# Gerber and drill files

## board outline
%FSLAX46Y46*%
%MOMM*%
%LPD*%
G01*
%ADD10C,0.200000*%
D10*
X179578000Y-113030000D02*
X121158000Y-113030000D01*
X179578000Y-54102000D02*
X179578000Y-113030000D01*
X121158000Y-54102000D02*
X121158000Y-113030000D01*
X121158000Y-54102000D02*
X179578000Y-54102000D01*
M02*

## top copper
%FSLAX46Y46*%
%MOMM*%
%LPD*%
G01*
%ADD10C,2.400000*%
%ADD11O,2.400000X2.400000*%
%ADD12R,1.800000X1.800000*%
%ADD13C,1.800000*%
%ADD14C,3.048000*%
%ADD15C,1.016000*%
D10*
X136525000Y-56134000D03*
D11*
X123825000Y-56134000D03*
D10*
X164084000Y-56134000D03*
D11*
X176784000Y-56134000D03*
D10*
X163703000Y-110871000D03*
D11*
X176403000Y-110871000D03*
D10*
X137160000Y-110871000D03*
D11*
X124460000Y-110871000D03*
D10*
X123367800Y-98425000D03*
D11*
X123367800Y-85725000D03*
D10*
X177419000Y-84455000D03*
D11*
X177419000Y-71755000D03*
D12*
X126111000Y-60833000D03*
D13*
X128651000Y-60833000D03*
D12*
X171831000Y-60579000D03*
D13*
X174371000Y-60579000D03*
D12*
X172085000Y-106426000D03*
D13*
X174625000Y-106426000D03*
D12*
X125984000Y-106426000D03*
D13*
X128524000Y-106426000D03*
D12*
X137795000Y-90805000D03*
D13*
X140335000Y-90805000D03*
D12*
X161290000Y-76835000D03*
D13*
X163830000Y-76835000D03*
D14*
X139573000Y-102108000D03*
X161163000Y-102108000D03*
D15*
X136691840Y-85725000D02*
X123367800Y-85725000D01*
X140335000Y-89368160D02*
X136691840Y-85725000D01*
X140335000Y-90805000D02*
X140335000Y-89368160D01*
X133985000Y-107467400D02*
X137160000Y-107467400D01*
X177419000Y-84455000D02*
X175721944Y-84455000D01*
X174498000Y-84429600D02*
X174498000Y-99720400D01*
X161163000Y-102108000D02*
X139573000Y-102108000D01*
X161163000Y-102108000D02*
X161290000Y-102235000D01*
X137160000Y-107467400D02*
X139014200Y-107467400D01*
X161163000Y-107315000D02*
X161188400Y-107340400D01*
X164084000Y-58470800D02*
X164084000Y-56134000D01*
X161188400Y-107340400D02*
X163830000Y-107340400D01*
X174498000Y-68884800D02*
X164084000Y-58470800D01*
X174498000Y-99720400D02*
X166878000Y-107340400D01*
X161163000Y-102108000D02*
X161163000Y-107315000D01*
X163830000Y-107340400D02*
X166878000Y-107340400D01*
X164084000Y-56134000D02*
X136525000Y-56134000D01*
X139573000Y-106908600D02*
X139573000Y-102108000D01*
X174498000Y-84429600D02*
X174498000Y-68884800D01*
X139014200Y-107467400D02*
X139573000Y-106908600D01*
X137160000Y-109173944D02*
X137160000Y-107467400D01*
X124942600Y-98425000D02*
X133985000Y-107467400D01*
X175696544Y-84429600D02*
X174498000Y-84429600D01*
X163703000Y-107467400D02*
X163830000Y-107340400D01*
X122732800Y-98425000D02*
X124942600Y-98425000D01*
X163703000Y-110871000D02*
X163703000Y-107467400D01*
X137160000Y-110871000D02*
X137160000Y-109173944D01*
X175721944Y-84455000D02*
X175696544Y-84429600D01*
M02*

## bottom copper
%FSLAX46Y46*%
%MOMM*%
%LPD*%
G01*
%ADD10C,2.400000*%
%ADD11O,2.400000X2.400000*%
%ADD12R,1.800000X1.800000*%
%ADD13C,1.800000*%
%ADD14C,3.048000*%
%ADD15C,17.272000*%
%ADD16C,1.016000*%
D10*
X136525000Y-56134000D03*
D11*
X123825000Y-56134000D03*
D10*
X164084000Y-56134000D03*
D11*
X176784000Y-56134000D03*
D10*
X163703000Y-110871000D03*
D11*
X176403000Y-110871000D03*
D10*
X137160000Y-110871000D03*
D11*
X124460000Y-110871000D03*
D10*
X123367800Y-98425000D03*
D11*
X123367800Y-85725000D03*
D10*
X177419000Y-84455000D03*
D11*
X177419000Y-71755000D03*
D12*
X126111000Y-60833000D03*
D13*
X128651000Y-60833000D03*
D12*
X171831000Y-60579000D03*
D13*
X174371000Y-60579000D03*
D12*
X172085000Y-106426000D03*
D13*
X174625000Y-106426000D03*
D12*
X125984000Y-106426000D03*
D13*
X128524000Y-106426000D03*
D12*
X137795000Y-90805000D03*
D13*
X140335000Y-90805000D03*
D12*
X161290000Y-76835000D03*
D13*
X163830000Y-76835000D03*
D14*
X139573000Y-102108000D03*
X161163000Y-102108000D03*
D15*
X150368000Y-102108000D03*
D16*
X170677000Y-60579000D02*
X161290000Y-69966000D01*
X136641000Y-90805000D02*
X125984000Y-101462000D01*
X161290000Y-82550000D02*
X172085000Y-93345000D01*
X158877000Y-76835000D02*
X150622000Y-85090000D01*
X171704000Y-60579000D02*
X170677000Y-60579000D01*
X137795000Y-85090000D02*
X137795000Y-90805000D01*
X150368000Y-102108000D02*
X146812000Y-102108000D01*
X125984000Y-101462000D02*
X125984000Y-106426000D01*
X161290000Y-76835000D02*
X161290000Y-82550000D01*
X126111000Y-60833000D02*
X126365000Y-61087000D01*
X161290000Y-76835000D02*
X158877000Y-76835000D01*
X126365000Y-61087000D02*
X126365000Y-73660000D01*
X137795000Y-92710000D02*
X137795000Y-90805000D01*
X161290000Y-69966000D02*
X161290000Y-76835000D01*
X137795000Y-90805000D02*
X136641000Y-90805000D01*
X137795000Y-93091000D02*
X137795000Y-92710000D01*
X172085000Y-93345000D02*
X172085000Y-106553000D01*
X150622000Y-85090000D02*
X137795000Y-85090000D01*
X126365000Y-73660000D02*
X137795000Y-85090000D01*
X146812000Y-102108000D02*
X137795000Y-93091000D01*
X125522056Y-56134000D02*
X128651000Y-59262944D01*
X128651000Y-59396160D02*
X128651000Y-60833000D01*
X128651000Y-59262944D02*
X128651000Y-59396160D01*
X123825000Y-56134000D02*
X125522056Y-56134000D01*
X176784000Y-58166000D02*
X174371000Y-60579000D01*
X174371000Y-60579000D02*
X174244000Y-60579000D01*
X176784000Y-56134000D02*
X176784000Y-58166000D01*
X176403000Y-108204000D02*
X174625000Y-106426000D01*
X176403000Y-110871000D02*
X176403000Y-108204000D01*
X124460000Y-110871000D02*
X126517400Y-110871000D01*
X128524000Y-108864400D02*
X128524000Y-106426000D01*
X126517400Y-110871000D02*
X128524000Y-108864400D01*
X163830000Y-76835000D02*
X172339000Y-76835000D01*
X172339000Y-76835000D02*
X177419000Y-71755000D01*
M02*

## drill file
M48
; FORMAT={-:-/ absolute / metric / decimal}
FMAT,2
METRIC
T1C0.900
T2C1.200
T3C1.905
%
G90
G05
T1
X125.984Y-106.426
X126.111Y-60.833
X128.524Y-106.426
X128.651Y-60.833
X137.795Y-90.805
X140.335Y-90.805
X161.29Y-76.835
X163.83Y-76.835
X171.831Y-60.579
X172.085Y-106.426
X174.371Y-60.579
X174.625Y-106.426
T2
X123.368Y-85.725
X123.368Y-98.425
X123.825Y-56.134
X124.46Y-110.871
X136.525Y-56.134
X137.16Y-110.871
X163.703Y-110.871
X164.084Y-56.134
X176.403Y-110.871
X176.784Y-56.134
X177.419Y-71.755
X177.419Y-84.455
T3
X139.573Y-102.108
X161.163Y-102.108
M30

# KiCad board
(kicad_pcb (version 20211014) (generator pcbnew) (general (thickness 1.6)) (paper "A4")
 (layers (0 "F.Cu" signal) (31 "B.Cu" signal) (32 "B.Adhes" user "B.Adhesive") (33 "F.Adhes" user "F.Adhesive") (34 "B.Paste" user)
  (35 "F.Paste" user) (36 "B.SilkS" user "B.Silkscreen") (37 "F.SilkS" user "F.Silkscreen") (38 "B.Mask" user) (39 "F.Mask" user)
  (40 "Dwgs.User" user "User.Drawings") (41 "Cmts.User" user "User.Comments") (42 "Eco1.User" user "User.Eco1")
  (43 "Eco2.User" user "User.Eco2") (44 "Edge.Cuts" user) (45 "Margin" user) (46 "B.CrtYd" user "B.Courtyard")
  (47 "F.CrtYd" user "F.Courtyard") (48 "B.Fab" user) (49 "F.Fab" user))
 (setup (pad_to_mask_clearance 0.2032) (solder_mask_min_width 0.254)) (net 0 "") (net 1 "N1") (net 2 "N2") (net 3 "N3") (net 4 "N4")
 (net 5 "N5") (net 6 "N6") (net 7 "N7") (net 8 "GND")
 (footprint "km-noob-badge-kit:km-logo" (layer "F.Cu") (at 150.368 83.566)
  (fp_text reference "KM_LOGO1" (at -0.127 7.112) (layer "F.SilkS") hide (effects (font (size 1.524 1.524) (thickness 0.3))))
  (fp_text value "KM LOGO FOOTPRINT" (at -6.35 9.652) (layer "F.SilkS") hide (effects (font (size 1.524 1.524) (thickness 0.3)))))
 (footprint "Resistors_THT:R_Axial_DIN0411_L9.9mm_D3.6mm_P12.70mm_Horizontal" (layer "F.Cu") (at 136.525 56.134 180)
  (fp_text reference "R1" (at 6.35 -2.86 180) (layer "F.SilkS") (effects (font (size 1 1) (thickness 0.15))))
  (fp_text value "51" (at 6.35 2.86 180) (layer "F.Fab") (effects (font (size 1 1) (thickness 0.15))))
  (pad "1" thru_hole circle locked (at 0 0 180) (size 2.4 2.4) (drill 1.2) (layers *.Cu *.Mask) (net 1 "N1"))
  (pad "2" thru_hole oval locked (at 12.7 0 180) (size 2.4 2.4) (drill 1.2) (layers *.Cu *.Mask) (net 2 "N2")))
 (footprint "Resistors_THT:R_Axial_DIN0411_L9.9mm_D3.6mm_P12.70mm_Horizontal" (layer "F.Cu") (at 164.084 56.134)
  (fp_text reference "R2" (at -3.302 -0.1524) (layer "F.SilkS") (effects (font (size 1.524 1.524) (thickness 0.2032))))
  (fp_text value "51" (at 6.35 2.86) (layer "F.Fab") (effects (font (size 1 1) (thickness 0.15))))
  (pad "1" thru_hole circle locked (at 0 0) (size 2.4 2.4) (drill 1.2) (layers *.Cu *.Mask) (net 1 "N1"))
  (pad "2" thru_hole oval locked (at 12.7 0) (size 2.4 2.4) (drill 1.2) (layers *.Cu *.Mask) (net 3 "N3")))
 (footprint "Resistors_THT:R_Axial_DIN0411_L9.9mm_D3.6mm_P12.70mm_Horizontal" (layer "F.Cu") (at 163.703 110.871)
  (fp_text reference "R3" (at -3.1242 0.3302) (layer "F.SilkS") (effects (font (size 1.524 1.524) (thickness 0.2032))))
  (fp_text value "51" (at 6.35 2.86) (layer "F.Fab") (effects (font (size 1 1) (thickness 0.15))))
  (pad "1" thru_hole circle locked (at 0 0) (size 2.4 2.4) (drill 1.2) (layers *.Cu *.Mask) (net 1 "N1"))
  (pad "2" thru_hole oval locked (at 12.7 0) (size 2.4 2.4) (drill 1.2) (layers *.Cu *.Mask) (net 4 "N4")))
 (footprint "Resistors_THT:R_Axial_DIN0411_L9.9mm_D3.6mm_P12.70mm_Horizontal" (layer "F.Cu") (at 137.16 110.871 180)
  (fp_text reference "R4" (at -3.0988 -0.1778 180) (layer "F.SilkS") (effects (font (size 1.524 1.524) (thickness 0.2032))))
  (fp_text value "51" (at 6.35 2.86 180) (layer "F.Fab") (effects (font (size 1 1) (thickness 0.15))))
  (pad "1" thru_hole circle locked (at 0 0 180) (size 2.4 2.4) (drill 1.2) (layers *.Cu *.Mask) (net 1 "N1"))
  (pad "2" thru_hole oval locked (at 12.7 0 180) (size 2.4 2.4) (drill 1.2) (layers *.Cu *.Mask) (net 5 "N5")))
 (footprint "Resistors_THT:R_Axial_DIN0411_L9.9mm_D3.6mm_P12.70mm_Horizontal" (layer "F.Cu") (at 123.3678 98.425 90)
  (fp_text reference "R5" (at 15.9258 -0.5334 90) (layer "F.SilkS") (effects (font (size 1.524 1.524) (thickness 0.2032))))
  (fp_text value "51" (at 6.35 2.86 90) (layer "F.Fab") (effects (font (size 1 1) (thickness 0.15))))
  (pad "1" thru_hole circle locked (at 0 0 90) (size 2.4 2.4) (drill 1.2) (layers *.Cu *.Mask) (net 1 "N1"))
  (pad "2" thru_hole oval locked (at 12.7 0 90) (size 2.4 2.4) (drill 1.2) (layers *.Cu *.Mask) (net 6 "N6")))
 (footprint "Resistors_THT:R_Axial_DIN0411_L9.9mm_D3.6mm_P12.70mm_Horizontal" (layer "F.Cu") (at 177.419 84.455 90)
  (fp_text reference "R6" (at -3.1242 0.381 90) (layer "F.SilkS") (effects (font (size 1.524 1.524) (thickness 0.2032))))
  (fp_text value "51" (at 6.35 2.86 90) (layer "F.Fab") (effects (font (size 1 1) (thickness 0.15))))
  (pad "1" thru_hole circle locked (at 0 0 90) (size 2.4 2.4) (drill 1.2) (layers *.Cu *.Mask) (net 1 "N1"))
  (pad "2" thru_hole oval locked (at 12.7 0 90) (size 2.4 2.4) (drill 1.2) (layers *.Cu *.Mask) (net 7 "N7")))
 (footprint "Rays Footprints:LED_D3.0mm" (layer "F.Cu") (at 126.111 60.833)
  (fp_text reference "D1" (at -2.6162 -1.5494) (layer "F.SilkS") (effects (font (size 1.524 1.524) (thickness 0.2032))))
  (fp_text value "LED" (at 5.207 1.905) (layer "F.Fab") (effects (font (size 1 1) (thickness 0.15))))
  (pad "1" thru_hole rect locked (at 0 0) (size 1.8 1.8) (drill 0.9) (layers *.Cu *.Mask) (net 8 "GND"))
  (pad "2" thru_hole circle locked (at 2.54 0) (size 1.8 1.8) (drill 0.9) (layers *.Cu *.Mask) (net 2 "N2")))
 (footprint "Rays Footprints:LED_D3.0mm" (layer "F.Cu") (at 171.831 60.579)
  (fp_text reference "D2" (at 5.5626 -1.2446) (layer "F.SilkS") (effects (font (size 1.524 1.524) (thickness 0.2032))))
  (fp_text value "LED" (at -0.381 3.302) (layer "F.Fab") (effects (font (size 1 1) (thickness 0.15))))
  (pad "1" thru_hole rect locked (at 0 0) (size 1.8 1.8) (drill 0.9) (layers *.Cu *.Mask) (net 8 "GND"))
  (pad "2" thru_hole circle locked (at 2.54 0) (size 1.8 1.8) (drill 0.9) (layers *.Cu *.Mask) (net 3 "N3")))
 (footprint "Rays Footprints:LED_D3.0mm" (layer "F.Cu") (at 172.085 106.426)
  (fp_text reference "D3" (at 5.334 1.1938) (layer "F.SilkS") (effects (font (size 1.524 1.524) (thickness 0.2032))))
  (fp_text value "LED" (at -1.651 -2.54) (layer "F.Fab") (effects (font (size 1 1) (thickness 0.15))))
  (pad "1" thru_hole rect locked (at 0 0) (size 1.8 1.8) (drill 0.9) (layers *.Cu *.Mask) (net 8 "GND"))
  (pad "2" thru_hole circle locked (at 2.54 0) (size 1.8 1.8) (drill 0.9) (layers *.Cu *.Mask) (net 4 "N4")))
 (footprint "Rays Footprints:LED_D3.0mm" (layer "F.Cu") (at 125.984 106.426)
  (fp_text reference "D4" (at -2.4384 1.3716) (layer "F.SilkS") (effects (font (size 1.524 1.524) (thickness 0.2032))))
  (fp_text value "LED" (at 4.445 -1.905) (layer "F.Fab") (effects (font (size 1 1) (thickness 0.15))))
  (pad "1" thru_hole rect locked (at 0 0) (size 1.8 1.8) (drill 0.9) (layers *.Cu *.Mask) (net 8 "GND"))
  (pad "2" thru_hole circle locked (at 2.54 0) (size 1.8 1.8) (drill 0.9) (layers *.Cu *.Mask) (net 5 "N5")))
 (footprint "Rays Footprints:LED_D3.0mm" (layer "F.Cu") (at 137.795 90.805)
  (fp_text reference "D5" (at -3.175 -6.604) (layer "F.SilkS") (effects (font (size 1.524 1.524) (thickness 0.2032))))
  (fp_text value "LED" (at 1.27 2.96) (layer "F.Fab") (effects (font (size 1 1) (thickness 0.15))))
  (pad "1" thru_hole rect locked (at 0 0) (size 1.8 1.8) (drill 0.9) (layers *.Cu *.Mask) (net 8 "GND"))
  (pad "2" thru_hole circle locked (at 2.54 0) (size 1.8 1.8) (drill 0.9) (layers *.Cu *.Mask) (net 6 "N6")))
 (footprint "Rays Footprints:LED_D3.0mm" (layer "F.Cu") (at 161.29 76.835)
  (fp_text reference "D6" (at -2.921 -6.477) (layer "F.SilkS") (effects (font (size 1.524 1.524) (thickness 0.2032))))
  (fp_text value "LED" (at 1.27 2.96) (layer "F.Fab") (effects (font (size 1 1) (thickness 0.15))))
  (pad "1" thru_hole rect locked (at 0 0) (size 1.8 1.8) (drill 0.9) (layers *.Cu *.Mask) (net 8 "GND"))
  (pad "2" thru_hole circle locked (at 2.54 0) (size 1.8 1.8) (drill 0.9) (layers *.Cu *.Mask) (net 7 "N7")))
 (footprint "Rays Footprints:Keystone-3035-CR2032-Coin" (layer "B.Cu") (at 150.368 102.108 180)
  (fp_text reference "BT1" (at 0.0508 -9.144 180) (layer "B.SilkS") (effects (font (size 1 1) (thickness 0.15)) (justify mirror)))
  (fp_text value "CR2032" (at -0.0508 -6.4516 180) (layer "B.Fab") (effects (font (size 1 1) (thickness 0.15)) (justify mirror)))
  (pad "1" thru_hole circle locked (at 10.795 0 180) (size 3.048 3.048) (drill 1.905) (layers *.Cu *.Mask) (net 1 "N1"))
  (pad "1" thru_hole circle locked (at -10.795 0 90) (size 3.048 3.048) (drill 1.905) (layers *.Cu *.Mask) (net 1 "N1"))
  (pad "2" smd circle locked (at 0 0 180) (size 17.272 17.272) (layers "B.Cu" "B.Paste" "B.Mask") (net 8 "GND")))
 (gr_line (start 179.578 113.03) (end 121.158 113.03) (layer "Edge.Cuts") (width 0.2))
 (gr_line (start 179.578 54.102) (end 179.578 113.03) (layer "Edge.Cuts") (width 0.2))
 (gr_line (start 121.158 54.102) (end 121.158 113.03) (layer "Edge.Cuts") (width 0.2))
 (gr_line (start 121.158 54.102) (end 179.578 54.102) (layer "Edge.Cuts") (width 0.2))
 (segment (start 170.677 60.579) (end 161.29 69.966) (width 1.016) (layer "B.Cu") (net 8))
 (segment (start 136.641 90.805) (end 125.984 101.462) (width 1.016) (layer "B.Cu") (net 8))
 (segment (start 161.29 82.55) (end 172.085 93.345) (width 1.016) (layer "B.Cu") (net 8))
 (segment (start 158.877 76.835) (end 150.622 85.09) (width 1.016) (layer "B.Cu") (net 8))
 (segment (start 171.704 60.579) (end 170.677 60.579) (width 1.016) (layer "B.Cu") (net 8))
 (segment (start 137.795 85.09) (end 137.795 90.805) (width 1.016) (layer "B.Cu") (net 8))
 (segment (start 150.368 102.108) (end 146.812 102.108) (width 1.016) (layer "B.Cu") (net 8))
 (segment (start 125.984 101.462) (end 125.984 106.426) (width 1.016) (layer "B.Cu") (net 8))
 (segment (start 161.29 76.835) (end 161.29 82.55) (width 1.016) (layer "B.Cu") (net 8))
 (segment (start 126.111 60.833) (end 126.365 61.087) (width 1.016) (layer "B.Cu") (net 8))
 (segment (start 161.29 76.835) (end 158.877 76.835) (width 1.016) (layer "B.Cu") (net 8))
 (segment (start 126.365 61.087) (end 126.365 73.66) (width 1.016) (layer "B.Cu") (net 8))
 (segment (start 137.795 92.71) (end 137.795 90.805) (width 1.016) (layer "B.Cu") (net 8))
 (segment (start 161.29 69.966) (end 161.29 76.835) (width 1.016) (layer "B.Cu") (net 8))
 (segment (start 137.795 90.805) (end 136.641 90.805) (width 1.016) (layer "B.Cu") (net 8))
 (segment (start 137.795 93.091) (end 137.795 92.71) (width 1.016) (layer "B.Cu") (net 8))
 (segment (start 172.085 93.345) (end 172.085 106.553) (width 1.016) (layer "B.Cu") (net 8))
 (segment (start 150.622 85.09) (end 137.795 85.09) (width 1.016) (layer "B.Cu") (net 8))
 (segment (start 126.365 73.66) (end 137.795 85.09) (width 1.016) (layer "B.Cu") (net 8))
 (segment (start 146.812 102.108) (end 137.795 93.091) (width 1.016) (layer "B.Cu") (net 8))
 (segment (start 125.522056 56.134) (end 128.651 59.262944) (width 1.016) (layer "B.Cu") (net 2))
 (segment (start 128.651 59.39616) (end 128.651 60.833) (width 1.016) (layer "B.Cu") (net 2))
 (segment (start 128.651 59.262944) (end 128.651 59.39616) (width 1.016) (layer "B.Cu") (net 2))
 (segment (start 123.825 56.134) (end 125.522056 56.134) (width 1.016) (layer "B.Cu") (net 2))
 (segment (start 176.784 58.166) (end 174.371 60.579) (width 1.016) (layer "B.Cu") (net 3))
 (segment (start 174.371 60.579) (end 174.244 60.579) (width 1.016) (layer "B.Cu") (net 3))
 (segment (start 176.784 56.134) (end 176.784 58.166) (width 1.016) (layer "B.Cu") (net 3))
 (segment (start 176.403 108.204) (end 174.625 106.426) (width 1.016) (layer "B.Cu") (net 4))
 (segment (start 176.403 110.871) (end 176.403 108.204) (width 1.016) (layer "B.Cu") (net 4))
 (segment (start 124.46 110.871) (end 126.5174 110.871) (width 1.016) (layer "B.Cu") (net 5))
 (segment (start 128.524 108.8644) (end 128.524 106.426) (width 1.016) (layer "B.Cu") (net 5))
 (segment (start 126.5174 110.871) (end 128.524 108.8644) (width 1.016) (layer "B.Cu") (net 5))
 (segment (start 136.69184 85.725) (end 123.3678 85.725) (width 1.016) (layer "F.Cu") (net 6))
 (segment (start 140.335 89.36816) (end 136.69184 85.725) (width 1.016) (layer "F.Cu") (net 6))
 (segment (start 140.335 90.805) (end 140.335 89.36816) (width 1.016) (layer "F.Cu") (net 6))
 (segment (start 163.83 76.835) (end 172.339 76.835) (width 1.016) (layer "B.Cu") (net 7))
 (segment (start 172.339 76.835) (end 177.419 71.755) (width 1.016) (layer "B.Cu") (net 7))
 (segment (start 133.985 107.4674) (end 137.16 107.4674) (width 1.016) (layer "F.Cu") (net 1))
 (segment (start 177.419 84.455) (end 175.721944 84.455) (width 1.016) (layer "F.Cu") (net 1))
 (segment (start 174.498 84.4296) (end 174.498 99.7204) (width 1.016) (layer "F.Cu") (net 1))
 (segment (start 161.163 102.108) (end 139.573 102.108) (width 1.016) (layer "F.Cu") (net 1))
 (segment (start 161.163 102.108) (end 161.29 102.235) (width 1.016) (layer "F.Cu") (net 1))
 (segment (start 137.16 107.4674) (end 139.0142 107.4674) (width 1.016) (layer "F.Cu") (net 1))
 (segment (start 161.163 107.315) (end 161.1884 107.3404) (width 1.016) (layer "F.Cu") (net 1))
 (segment (start 164.084 58.4708) (end 164.084 56.134) (width 1.016) (layer "F.Cu") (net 1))
 (segment (start 161.1884 107.3404) (end 163.83 107.3404) (width 1.016) (layer "F.Cu") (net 1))
 (segment (start 174.498 68.8848) (end 164.084 58.4708) (width 1.016) (layer "F.Cu") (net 1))
 (segment (start 174.498 99.7204) (end 166.878 107.3404) (width 1.016) (layer "F.Cu") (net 1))
 (segment (start 161.163 102.108) (end 161.163 107.315) (width 1.016) (layer "F.Cu") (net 1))
 (segment (start 163.83 107.3404) (end 166.878 107.3404) (width 1.016) (layer "F.Cu") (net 1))
 (segment (start 164.084 56.134) (end 136.525 56.134) (width 1.016) (layer "F.Cu") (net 1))
 (segment (start 139.573 106.9086) (end 139.573 102.108) (width 1.016) (layer "F.Cu") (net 1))
 (segment (start 174.498 84.4296) (end 174.498 68.8848) (width 1.016) (layer "F.Cu") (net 1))
 (segment (start 139.0142 107.4674) (end 139.573 106.9086) (width 1.016) (layer "F.Cu") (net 1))
 (segment (start 137.16 109.173944) (end 137.16 107.4674) (width 1.016) (layer "F.Cu") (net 1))
 (segment (start 124.9426 98.425) (end 133.985 107.4674) (width 1.016) (layer "F.Cu") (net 1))
 (segment (start 175.696544 84.4296) (end 174.498 84.4296) (width 1.016) (layer "F.Cu") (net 1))
 (segment (start 163.703 107.4674) (end 163.83 107.3404) (width 1.016) (layer "F.Cu") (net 1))
 (segment (start 122.7328 98.425) (end 124.9426 98.425) (width 1.016) (layer "F.Cu") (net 1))
 (segment (start 163.703 110.871) (end 163.703 107.4674) (width 1.016) (layer "F.Cu") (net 1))
 (segment (start 137.16 110.871) (end 137.16 109.173944) (width 1.016) (layer "F.Cu") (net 1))
 (segment (start 175.721944 84.455) (end 175.696544 84.4296) (width 1.016) (layer "F.Cu") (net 1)))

